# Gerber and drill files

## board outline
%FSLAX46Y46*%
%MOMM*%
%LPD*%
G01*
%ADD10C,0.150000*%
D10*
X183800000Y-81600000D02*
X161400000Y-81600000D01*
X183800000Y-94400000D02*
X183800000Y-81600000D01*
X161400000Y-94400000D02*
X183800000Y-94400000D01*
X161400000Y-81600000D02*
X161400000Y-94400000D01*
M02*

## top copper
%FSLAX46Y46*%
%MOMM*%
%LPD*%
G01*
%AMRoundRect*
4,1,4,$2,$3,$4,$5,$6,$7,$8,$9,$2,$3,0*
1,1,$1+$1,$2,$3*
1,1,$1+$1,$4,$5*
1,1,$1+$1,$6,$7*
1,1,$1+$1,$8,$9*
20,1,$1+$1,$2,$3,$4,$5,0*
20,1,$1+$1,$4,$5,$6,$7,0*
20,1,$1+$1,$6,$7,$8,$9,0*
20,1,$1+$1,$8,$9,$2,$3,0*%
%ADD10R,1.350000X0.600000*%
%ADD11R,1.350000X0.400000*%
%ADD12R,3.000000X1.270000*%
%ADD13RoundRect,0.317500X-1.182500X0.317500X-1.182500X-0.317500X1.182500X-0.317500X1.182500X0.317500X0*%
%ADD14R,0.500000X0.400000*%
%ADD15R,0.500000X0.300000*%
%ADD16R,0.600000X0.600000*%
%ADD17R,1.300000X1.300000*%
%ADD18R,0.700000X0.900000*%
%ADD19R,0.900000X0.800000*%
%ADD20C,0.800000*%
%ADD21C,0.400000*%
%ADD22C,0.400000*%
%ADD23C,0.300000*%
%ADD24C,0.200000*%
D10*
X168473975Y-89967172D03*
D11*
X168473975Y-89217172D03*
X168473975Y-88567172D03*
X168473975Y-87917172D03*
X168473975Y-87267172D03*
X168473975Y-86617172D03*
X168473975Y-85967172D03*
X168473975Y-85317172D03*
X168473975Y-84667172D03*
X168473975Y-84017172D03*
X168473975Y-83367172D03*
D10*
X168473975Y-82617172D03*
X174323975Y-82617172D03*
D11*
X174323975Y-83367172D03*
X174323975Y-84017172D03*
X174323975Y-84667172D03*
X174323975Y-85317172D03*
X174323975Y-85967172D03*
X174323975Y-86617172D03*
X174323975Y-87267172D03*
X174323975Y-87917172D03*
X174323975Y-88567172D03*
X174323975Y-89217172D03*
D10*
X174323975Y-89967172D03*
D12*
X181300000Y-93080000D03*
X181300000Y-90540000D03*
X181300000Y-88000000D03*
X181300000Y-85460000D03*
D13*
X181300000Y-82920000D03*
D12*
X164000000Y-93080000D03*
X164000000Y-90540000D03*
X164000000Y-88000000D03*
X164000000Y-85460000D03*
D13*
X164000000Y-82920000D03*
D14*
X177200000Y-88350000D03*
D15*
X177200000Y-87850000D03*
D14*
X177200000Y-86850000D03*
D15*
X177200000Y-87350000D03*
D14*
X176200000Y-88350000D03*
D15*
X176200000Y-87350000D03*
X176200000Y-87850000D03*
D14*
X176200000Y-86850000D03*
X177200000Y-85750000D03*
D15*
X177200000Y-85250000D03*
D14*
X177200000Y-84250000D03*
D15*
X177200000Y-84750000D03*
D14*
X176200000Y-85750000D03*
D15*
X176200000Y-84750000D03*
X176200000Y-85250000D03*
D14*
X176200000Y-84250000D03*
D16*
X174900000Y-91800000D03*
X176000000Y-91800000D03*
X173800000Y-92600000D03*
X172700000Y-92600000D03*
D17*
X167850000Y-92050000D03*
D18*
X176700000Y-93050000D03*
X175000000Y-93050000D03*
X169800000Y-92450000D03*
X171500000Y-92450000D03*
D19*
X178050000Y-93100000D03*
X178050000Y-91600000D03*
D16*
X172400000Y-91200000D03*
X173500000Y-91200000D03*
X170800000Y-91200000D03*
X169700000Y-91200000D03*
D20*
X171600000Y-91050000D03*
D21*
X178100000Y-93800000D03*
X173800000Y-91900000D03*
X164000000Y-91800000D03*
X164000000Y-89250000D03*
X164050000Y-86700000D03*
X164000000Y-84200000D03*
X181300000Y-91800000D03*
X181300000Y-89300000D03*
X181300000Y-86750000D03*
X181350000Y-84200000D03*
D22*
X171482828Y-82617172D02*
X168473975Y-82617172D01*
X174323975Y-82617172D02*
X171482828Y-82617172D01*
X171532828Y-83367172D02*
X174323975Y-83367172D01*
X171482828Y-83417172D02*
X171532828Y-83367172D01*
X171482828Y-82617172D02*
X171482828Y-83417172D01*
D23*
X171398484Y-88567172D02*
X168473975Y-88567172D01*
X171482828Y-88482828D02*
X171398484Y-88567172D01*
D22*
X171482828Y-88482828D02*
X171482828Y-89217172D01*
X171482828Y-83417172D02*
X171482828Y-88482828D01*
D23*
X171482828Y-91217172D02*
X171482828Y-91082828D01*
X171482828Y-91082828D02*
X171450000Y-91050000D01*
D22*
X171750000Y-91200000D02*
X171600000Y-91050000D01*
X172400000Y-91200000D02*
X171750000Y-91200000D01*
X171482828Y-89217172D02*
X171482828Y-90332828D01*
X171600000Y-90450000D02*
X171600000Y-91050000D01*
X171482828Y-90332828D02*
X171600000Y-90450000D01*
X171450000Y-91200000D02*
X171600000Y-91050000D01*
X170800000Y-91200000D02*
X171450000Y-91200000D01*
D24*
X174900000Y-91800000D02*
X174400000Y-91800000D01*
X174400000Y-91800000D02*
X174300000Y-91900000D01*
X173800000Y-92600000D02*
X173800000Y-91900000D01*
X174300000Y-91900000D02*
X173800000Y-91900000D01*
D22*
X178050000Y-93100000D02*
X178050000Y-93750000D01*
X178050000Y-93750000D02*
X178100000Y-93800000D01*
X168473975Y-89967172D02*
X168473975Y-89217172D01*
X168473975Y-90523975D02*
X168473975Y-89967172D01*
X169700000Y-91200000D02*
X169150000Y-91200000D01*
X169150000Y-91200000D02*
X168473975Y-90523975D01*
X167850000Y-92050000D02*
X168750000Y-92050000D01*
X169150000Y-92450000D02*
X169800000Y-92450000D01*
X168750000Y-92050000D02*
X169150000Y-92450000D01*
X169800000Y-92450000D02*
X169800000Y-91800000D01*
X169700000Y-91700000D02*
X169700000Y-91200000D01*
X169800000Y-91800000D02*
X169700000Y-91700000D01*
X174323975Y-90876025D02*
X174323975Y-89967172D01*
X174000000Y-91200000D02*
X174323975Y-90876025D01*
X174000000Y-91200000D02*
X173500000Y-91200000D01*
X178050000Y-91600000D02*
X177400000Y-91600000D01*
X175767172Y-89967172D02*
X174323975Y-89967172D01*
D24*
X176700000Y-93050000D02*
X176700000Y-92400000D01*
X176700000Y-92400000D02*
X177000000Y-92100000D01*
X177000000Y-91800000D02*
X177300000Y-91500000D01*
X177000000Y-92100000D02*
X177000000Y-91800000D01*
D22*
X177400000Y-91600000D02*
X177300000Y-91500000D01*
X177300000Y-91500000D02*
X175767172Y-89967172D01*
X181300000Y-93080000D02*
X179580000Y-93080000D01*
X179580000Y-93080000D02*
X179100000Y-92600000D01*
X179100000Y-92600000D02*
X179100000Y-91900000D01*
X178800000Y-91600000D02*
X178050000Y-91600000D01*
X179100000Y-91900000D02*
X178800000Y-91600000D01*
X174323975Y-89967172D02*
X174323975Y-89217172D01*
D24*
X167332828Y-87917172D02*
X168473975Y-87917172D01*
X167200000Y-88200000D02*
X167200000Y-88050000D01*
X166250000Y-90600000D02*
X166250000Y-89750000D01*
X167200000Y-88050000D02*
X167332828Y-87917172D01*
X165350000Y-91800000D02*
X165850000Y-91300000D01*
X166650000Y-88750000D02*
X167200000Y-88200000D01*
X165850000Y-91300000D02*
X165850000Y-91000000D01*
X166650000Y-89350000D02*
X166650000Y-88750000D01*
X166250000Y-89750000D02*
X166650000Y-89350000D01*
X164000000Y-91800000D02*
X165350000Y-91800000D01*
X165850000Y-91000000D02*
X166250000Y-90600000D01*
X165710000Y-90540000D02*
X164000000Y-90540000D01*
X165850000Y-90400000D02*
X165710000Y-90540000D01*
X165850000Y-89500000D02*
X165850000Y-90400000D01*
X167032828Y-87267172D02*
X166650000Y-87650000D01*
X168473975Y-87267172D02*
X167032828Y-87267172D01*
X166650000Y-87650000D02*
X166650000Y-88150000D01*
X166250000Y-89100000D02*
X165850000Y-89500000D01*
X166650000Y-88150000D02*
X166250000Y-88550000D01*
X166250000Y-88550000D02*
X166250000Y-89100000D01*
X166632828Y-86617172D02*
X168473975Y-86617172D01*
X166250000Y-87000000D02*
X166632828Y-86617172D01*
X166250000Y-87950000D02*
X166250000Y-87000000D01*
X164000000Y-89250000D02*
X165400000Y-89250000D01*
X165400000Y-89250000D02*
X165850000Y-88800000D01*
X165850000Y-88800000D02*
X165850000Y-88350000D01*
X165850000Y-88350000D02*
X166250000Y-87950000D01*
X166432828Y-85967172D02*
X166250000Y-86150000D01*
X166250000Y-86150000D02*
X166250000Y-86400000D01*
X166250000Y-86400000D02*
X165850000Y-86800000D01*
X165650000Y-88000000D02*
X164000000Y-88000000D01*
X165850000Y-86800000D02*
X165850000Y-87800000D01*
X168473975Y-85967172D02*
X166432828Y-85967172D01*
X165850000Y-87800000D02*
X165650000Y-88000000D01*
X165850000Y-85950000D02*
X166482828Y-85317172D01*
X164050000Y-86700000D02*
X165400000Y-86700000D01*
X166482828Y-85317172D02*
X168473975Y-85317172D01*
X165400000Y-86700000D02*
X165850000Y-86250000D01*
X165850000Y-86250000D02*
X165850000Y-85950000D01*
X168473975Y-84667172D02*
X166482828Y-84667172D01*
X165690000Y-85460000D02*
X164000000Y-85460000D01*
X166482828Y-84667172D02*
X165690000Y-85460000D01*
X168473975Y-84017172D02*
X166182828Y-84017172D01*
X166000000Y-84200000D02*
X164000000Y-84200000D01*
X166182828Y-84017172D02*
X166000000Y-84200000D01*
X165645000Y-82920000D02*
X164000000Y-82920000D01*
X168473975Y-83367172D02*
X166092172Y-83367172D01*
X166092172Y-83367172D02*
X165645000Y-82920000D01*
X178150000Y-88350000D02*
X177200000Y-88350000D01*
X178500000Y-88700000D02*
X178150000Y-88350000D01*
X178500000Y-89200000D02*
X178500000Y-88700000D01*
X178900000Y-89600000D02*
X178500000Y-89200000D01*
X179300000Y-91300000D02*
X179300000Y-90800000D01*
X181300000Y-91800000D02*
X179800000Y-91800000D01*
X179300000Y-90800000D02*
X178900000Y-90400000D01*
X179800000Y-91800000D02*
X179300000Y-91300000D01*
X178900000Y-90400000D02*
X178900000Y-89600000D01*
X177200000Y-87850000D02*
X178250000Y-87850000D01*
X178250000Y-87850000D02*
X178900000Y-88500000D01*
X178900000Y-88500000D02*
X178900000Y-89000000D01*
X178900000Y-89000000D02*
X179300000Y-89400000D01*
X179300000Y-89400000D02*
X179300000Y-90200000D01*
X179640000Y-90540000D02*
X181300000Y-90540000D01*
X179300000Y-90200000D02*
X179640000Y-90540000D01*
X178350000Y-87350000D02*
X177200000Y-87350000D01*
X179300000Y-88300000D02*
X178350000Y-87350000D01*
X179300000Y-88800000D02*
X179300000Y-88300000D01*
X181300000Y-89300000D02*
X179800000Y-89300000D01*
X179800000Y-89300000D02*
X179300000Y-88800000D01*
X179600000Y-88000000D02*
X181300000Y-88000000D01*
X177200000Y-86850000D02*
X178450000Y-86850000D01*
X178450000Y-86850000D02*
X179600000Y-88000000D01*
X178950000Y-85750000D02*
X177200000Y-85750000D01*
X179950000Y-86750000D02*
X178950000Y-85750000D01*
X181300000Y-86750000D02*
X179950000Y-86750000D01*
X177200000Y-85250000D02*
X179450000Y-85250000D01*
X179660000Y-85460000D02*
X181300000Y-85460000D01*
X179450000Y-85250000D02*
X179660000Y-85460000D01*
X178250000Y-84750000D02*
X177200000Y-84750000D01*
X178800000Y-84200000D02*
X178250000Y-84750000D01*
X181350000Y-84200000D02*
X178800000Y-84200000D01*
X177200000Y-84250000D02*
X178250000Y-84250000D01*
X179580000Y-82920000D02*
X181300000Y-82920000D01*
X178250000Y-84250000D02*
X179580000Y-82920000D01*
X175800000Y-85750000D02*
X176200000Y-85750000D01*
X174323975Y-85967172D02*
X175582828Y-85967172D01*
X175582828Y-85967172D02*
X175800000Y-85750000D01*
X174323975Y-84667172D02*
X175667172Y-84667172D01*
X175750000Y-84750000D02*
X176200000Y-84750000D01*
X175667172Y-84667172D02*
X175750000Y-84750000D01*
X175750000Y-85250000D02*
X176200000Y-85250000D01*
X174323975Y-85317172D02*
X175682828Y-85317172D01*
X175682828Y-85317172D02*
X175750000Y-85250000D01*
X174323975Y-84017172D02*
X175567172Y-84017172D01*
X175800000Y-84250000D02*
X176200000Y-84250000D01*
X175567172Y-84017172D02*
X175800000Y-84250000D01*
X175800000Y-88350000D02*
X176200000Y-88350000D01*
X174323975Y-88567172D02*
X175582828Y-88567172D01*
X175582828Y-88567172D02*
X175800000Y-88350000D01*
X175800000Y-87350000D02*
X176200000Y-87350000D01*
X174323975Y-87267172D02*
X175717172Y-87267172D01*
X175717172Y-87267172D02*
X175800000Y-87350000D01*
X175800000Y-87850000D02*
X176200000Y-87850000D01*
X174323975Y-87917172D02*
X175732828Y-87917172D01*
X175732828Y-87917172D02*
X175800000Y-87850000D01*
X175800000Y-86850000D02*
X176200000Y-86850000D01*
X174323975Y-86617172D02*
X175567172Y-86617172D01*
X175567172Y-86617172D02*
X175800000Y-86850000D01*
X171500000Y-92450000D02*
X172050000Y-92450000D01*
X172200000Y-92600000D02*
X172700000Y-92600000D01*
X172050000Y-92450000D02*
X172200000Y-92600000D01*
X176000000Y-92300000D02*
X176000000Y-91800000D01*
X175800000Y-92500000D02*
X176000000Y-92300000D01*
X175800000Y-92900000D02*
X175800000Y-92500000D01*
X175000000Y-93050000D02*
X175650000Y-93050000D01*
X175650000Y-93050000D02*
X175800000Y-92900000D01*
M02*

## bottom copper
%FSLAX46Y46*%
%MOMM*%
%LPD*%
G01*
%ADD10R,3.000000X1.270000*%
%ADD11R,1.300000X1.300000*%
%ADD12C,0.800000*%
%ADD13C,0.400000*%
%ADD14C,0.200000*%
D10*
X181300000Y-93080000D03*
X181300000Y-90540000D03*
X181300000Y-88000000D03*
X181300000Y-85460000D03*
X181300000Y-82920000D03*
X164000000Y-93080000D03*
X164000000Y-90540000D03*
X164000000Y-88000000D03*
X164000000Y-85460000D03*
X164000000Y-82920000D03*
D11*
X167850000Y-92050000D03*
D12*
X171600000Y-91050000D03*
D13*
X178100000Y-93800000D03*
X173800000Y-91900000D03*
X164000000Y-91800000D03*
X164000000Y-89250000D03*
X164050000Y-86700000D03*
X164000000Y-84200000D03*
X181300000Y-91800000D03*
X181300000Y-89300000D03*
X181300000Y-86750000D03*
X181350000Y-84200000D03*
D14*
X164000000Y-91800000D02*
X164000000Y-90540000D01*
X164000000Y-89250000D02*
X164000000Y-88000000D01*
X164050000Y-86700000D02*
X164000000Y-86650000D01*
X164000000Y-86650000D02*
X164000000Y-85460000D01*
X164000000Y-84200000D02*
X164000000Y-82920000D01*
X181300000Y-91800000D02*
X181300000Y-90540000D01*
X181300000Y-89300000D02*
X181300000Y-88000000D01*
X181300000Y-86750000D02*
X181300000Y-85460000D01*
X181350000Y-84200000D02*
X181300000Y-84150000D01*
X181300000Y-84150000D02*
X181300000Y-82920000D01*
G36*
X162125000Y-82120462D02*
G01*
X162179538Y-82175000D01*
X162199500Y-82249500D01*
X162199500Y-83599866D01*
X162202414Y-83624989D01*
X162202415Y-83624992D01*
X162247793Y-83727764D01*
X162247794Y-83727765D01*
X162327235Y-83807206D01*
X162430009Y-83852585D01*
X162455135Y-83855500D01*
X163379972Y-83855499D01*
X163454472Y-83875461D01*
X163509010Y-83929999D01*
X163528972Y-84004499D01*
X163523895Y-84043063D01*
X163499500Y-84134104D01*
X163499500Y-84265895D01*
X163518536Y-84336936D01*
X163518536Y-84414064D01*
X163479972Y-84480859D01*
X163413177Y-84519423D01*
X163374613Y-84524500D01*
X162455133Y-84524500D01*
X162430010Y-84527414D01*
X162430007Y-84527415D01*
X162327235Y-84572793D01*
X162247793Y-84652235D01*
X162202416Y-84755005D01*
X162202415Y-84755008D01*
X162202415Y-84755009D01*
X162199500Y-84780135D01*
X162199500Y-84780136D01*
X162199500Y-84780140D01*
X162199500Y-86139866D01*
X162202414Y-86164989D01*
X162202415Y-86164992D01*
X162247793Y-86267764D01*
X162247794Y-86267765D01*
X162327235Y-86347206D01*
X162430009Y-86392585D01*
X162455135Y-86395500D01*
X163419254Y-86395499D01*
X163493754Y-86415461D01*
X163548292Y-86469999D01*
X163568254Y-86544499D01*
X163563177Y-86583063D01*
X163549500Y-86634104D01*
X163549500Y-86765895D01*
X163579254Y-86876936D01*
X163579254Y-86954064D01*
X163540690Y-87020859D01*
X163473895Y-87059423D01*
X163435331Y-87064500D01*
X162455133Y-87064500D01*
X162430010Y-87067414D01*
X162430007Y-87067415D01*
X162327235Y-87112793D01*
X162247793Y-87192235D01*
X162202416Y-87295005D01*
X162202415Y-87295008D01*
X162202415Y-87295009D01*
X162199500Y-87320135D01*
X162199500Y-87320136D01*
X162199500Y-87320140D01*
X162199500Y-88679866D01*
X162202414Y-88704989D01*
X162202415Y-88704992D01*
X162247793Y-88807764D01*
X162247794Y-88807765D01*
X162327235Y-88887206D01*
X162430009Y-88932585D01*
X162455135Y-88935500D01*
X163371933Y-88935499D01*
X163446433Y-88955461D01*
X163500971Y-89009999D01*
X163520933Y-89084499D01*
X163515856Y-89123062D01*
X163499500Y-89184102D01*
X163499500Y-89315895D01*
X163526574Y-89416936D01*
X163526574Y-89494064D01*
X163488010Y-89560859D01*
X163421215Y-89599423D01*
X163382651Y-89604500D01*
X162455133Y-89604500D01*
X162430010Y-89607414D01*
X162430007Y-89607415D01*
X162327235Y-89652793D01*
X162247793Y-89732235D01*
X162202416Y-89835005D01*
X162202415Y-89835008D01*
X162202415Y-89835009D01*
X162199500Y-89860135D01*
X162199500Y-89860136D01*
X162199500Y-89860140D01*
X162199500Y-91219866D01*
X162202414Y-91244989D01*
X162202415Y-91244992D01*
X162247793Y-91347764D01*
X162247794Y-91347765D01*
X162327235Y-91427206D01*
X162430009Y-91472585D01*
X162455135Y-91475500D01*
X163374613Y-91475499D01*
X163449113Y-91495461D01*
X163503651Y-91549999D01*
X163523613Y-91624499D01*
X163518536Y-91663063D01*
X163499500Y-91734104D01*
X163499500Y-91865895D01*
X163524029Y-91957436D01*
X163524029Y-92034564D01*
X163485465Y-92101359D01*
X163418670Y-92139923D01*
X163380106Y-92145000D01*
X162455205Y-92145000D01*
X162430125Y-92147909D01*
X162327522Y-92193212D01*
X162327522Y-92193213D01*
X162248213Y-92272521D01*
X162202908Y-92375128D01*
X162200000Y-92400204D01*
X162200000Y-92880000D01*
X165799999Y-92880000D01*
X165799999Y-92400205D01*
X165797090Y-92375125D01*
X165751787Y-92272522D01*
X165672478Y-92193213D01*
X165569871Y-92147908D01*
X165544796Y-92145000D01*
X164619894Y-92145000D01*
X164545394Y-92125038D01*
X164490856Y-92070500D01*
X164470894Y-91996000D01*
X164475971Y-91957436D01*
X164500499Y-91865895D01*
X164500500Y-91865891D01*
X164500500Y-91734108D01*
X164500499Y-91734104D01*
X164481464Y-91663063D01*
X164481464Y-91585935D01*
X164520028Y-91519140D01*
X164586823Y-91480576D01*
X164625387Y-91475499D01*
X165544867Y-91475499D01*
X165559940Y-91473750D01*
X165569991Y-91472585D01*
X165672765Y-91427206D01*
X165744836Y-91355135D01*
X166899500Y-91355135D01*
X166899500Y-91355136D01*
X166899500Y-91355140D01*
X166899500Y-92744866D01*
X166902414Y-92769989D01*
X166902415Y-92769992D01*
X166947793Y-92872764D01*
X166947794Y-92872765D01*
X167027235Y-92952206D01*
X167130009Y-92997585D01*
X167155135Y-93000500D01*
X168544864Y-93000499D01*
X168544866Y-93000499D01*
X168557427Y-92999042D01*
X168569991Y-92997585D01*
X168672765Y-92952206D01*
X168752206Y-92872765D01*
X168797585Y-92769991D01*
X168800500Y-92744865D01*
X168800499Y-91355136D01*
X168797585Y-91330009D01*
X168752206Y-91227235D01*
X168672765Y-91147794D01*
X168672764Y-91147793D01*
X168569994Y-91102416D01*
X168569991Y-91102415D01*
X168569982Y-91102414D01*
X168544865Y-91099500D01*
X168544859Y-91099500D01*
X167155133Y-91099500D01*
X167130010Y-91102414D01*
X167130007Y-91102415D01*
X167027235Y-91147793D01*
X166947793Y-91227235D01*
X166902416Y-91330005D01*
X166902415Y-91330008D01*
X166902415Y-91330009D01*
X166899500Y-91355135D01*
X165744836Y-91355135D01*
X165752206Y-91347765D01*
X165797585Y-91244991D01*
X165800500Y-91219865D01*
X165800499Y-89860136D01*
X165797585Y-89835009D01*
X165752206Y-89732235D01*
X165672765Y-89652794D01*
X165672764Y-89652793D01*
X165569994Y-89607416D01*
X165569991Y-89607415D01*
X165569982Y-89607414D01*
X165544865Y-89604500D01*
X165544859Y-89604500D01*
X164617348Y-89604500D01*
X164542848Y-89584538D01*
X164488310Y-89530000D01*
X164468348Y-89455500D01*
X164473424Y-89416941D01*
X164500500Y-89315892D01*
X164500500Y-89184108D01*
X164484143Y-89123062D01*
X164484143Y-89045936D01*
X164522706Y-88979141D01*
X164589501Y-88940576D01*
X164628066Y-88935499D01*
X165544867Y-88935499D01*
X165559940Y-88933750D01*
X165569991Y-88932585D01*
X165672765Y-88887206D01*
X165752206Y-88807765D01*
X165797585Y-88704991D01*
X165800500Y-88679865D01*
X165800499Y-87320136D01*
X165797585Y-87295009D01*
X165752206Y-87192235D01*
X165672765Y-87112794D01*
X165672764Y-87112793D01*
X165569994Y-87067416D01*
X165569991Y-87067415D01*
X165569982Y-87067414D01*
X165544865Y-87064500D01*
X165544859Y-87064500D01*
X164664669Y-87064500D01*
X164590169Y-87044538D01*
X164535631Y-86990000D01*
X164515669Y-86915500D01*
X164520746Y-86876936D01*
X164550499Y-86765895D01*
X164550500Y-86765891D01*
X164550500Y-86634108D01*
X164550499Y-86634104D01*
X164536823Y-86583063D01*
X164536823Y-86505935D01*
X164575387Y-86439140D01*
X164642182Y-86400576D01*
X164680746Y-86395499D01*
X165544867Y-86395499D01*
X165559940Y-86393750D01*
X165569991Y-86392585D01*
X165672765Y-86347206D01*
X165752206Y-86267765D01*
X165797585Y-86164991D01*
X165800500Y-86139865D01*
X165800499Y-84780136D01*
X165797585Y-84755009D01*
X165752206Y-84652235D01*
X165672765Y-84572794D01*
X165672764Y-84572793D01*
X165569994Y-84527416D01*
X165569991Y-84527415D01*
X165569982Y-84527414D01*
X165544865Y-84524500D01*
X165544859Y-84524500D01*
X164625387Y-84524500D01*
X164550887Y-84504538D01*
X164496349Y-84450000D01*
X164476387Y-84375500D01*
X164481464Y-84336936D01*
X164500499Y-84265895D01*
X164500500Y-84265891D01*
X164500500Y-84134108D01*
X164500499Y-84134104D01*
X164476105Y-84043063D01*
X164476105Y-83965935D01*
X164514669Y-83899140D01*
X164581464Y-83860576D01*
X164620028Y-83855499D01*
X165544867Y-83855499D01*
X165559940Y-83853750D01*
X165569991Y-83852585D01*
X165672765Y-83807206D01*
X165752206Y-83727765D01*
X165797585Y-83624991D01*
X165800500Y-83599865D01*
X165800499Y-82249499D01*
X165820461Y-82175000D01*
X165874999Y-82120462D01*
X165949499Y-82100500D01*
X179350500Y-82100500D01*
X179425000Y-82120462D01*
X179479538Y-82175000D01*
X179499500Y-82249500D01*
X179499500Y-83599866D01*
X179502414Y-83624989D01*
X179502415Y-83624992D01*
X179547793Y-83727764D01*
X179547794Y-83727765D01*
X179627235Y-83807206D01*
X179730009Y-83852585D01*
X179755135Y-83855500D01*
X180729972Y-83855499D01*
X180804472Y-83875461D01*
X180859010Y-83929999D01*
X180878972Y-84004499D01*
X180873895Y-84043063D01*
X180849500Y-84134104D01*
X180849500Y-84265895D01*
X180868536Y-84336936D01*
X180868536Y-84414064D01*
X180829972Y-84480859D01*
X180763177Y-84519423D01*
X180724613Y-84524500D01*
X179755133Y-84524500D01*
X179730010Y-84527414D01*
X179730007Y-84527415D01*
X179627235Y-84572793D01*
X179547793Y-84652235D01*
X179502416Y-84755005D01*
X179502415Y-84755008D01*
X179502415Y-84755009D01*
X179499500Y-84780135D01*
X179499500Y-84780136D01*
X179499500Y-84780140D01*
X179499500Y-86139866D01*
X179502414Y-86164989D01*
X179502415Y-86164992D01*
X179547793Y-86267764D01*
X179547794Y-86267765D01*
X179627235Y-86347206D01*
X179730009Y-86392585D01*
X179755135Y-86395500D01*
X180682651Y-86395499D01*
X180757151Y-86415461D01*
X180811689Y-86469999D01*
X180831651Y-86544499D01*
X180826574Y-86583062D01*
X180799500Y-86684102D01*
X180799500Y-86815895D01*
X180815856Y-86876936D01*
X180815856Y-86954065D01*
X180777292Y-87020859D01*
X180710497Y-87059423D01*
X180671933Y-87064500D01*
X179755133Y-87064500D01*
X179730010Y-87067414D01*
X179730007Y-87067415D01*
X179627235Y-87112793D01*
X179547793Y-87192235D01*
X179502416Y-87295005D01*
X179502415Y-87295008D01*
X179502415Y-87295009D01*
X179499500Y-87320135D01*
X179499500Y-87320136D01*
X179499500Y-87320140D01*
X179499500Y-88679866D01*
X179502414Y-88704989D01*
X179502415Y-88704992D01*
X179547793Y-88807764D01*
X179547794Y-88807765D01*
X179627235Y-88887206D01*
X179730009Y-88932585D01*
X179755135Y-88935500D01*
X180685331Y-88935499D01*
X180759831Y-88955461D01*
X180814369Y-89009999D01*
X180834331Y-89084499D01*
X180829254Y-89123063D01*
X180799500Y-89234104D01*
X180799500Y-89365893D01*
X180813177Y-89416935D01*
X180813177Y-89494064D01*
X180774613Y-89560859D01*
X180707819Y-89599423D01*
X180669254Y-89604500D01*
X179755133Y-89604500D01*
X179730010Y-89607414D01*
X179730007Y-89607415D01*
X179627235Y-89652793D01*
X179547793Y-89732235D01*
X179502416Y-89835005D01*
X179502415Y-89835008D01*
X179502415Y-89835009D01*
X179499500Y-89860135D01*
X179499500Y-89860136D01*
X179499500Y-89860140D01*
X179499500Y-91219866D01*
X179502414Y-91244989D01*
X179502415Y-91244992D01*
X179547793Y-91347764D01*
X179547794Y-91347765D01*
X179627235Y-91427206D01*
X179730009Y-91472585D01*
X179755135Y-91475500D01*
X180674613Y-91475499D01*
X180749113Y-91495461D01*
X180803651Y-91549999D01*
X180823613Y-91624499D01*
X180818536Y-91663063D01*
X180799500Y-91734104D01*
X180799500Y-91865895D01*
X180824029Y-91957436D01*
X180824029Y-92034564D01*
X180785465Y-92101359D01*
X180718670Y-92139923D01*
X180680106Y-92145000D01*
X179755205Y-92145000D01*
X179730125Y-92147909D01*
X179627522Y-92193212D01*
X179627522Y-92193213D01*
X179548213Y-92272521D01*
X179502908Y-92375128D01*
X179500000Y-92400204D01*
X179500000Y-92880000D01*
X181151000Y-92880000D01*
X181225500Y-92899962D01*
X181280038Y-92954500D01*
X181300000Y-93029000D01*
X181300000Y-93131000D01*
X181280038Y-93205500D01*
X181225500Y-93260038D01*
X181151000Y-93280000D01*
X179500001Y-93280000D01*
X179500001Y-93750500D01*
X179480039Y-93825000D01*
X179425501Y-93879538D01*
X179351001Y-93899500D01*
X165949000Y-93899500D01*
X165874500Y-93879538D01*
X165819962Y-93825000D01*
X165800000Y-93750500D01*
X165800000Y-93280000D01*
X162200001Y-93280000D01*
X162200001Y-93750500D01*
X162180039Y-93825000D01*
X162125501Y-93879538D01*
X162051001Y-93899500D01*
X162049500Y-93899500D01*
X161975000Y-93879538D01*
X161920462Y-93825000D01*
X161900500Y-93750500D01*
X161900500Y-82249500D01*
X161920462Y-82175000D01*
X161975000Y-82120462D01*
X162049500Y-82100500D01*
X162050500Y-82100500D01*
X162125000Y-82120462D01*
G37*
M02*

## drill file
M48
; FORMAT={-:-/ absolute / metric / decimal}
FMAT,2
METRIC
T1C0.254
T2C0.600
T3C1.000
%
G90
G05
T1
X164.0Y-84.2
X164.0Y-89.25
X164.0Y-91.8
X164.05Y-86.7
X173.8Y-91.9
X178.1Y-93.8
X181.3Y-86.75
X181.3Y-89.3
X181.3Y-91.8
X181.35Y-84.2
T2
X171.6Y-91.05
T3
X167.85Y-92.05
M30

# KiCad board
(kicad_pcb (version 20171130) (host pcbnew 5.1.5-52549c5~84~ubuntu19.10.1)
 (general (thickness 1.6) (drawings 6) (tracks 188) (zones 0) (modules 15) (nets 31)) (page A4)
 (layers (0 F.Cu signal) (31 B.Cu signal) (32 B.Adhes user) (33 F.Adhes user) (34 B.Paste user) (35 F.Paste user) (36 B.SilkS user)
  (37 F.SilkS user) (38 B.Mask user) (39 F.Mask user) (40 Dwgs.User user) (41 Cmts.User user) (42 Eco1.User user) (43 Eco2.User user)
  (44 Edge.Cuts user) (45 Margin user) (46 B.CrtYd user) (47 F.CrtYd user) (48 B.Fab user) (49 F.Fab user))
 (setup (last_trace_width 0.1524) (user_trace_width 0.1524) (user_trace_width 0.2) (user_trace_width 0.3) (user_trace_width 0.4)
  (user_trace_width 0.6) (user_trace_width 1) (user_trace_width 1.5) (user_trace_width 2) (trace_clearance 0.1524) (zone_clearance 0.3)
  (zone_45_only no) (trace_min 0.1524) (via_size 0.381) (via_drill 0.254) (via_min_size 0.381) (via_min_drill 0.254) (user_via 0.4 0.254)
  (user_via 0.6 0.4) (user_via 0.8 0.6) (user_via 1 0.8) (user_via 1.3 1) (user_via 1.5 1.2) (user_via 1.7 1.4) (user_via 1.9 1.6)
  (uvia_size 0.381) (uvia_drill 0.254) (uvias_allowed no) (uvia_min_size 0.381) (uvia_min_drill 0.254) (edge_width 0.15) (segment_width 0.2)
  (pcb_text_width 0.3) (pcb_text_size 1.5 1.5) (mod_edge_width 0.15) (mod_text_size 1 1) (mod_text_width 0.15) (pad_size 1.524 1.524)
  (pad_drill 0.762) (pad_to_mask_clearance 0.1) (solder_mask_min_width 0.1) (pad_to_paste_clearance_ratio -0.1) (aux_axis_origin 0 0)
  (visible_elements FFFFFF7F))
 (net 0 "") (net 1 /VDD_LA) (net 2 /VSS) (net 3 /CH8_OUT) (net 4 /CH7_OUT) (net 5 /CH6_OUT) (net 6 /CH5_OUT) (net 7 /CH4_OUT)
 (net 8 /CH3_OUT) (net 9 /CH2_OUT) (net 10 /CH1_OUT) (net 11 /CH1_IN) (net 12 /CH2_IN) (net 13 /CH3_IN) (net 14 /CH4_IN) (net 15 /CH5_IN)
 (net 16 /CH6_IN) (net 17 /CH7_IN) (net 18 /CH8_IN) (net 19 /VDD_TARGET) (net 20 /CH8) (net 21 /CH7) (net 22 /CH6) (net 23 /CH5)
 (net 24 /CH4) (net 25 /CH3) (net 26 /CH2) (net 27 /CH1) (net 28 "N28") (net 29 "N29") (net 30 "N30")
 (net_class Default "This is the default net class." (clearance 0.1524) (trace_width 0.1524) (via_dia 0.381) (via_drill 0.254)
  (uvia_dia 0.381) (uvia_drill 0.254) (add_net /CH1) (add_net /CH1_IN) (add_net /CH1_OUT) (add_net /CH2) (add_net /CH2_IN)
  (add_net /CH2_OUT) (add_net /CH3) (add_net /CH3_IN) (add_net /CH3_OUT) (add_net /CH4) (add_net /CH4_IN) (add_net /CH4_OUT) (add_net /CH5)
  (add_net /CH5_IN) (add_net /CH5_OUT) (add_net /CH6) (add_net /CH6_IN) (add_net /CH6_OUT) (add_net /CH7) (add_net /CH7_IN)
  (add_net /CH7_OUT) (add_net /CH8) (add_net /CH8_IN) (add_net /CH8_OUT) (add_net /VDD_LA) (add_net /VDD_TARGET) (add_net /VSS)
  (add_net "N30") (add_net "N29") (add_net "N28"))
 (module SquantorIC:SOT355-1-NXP (layer F.Cu) (at 171.35 86.25 180)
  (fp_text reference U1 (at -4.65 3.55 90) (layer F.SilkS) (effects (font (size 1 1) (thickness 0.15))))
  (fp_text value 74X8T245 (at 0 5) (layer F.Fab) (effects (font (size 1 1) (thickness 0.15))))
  (pad 24 smd rect (at 2.876025 -3.717172 90) (size 0.6 1.35) (layers F.Cu F.Paste F.Mask) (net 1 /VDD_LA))
  (pad 23 smd rect (at 2.876025 -2.967172 90) (size 0.4 1.35) (layers F.Cu F.Paste F.Mask) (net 1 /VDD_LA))
  (pad 22 smd rect (at 2.876025 -2.317172 90) (size 0.4 1.35) (layers F.Cu F.Paste F.Mask) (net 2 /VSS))
  (pad 21 smd rect (at 2.876025 -1.667172 90) (size 0.4 1.35) (layers F.Cu F.Paste F.Mask) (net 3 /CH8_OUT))
  (pad 20 smd rect (at 2.876025 -1.017172 90) (size 0.4 1.35) (layers F.Cu F.Paste F.Mask) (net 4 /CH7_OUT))
  (pad 19 smd rect (at 2.876025 -0.367172 90) (size 0.4 1.35) (layers F.Cu F.Paste F.Mask) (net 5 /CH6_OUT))
  (pad 18 smd rect (at 2.876025 0.282828 90) (size 0.4 1.35) (layers F.Cu F.Paste F.Mask) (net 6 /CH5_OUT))
  (pad 17 smd rect (at 2.876025 0.932828 90) (size 0.4 1.35) (layers F.Cu F.Paste F.Mask) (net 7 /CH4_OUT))
  (pad 16 smd rect (at 2.876025 1.582828 90) (size 0.4 1.35) (layers F.Cu F.Paste F.Mask) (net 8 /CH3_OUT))
  (pad 15 smd rect (at 2.876025 2.232828 90) (size 0.4 1.35) (layers F.Cu F.Paste F.Mask) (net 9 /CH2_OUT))
  (pad 14 smd rect (at 2.876025 2.882828 90) (size 0.4 1.35) (layers F.Cu F.Paste F.Mask) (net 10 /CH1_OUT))
  (pad 13 smd rect (at 2.876025 3.632828 90) (size 0.6 1.35) (layers F.Cu F.Paste F.Mask) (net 2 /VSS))
  (pad 12 smd rect (at -2.973975 3.632828 90) (size 0.6 1.35) (layers F.Cu F.Paste F.Mask) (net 2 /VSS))
  (pad 11 smd rect (at -2.973975 2.882828 90) (size 0.4 1.35) (layers F.Cu F.Paste F.Mask) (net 2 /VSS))
  (pad 10 smd rect (at -2.973975 2.232828 90) (size 0.4 1.35) (layers F.Cu F.Paste F.Mask) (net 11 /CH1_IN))
  (pad 9 smd rect (at -2.973975 1.582828 90) (size 0.4 1.35) (layers F.Cu F.Paste F.Mask) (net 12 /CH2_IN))
  (pad 8 smd rect (at -2.973975 0.932828 90) (size 0.4 1.35) (layers F.Cu F.Paste F.Mask) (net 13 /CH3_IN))
  (pad 7 smd rect (at -2.973975 0.282828 90) (size 0.4 1.35) (layers F.Cu F.Paste F.Mask) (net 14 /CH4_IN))
  (pad 6 smd rect (at -2.973975 -0.367172 90) (size 0.4 1.35) (layers F.Cu F.Paste F.Mask) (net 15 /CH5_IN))
  (pad 5 smd rect (at -2.973975 -1.017172 90) (size 0.4 1.35) (layers F.Cu F.Paste F.Mask) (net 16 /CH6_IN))
  (pad 4 smd rect (at -2.973975 -1.667172 90) (size 0.4 1.35) (layers F.Cu F.Paste F.Mask) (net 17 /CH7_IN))
  (pad 3 smd rect (at -2.973975 -2.317172 90) (size 0.4 1.35) (layers F.Cu F.Paste F.Mask) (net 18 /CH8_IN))
  (pad 2 smd rect (at -2.973975 -2.967172 90) (size 0.4 1.35) (layers F.Cu F.Paste F.Mask) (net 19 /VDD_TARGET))
  (pad 1 smd rect (at -2.973975 -3.717172 90) (size 0.6 1.35) (layers F.Cu F.Paste F.Mask) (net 19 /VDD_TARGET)))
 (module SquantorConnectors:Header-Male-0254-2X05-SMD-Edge (layer B.Cu) (at 183.84 88 270)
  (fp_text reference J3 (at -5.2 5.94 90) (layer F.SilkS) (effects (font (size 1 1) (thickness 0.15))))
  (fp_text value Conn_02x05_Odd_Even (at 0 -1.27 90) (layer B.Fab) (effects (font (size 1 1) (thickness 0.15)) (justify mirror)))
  (pad 10 smd rect (at 5.08 2.54 270) (size 1.27 3) (layers B.Cu B.Paste B.Mask) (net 2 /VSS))
  (pad 9 smd rect (at 5.08 2.54 270) (size 1.27 3) (layers F.Cu F.Paste F.Mask) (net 19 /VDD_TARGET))
  (pad 8 smd rect (at 2.54 2.54 270) (size 1.27 3) (layers B.Cu B.Paste B.Mask) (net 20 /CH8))
  (pad 7 smd rect (at 2.54 2.54 270) (size 1.27 3) (layers F.Cu F.Paste F.Mask) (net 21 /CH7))
  (pad 6 smd rect (at 0 2.54 270) (size 1.27 3) (layers B.Cu B.Paste B.Mask) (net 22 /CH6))
  (pad 5 smd rect (at 0 2.54 270) (size 1.27 3) (layers F.Cu F.Paste F.Mask) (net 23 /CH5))
  (pad 4 smd rect (at -2.54 2.54 270) (size 1.27 3) (layers B.Cu B.Paste B.Mask) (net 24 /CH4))
  (pad 3 smd rect (at -2.54 2.54 270) (size 1.27 3) (layers F.Cu F.Paste F.Mask) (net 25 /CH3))
  (pad 2 smd rect (at -5.08 2.54 270) (size 1.27 3) (layers B.Cu B.Paste B.Mask) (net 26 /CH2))
  (pad 1 smd roundrect (at -5.08 2.54 270) (size 1.27 3) (layers F.Cu F.Paste F.Mask) (roundrect_rratio 0.25) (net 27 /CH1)))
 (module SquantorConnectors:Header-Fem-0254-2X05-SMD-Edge (layer F.Cu) (at 161.46 88 270)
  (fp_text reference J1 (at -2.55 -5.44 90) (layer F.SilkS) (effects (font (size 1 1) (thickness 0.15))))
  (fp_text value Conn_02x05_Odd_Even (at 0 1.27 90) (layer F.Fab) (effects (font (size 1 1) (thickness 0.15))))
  (pad 10 smd rect (at 5.08 -2.54 270) (size 1.27 3) (layers B.Cu B.Paste B.Mask) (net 2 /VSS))
  (pad 9 smd rect (at 5.08 -2.54 270) (size 1.27 3) (layers F.Cu F.Paste F.Mask) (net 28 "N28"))
  (pad 8 smd rect (at 2.54 -2.54 270) (size 1.27 3) (layers B.Cu B.Paste B.Mask) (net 3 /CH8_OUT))
  (pad 7 smd rect (at 2.54 -2.54 270) (size 1.27 3) (layers F.Cu F.Paste F.Mask) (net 4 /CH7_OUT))
  (pad 6 smd rect (at 0 -2.54 270) (size 1.27 3) (layers B.Cu B.Paste B.Mask) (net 5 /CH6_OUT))
  (pad 5 smd rect (at 0 -2.54 270) (size 1.27 3) (layers F.Cu F.Paste F.Mask) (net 6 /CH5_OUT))
  (pad 4 smd rect (at -2.54 -2.54 270) (size 1.27 3) (layers B.Cu B.Paste B.Mask) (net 7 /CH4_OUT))
  (pad 3 smd rect (at -2.54 -2.54 270) (size 1.27 3) (layers F.Cu F.Paste F.Mask) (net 8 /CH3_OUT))
  (pad 2 smd rect (at -5.08 -2.54 270) (size 1.27 3) (layers B.Cu B.Paste B.Mask) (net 9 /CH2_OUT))
  (pad 1 smd roundrect (at -5.08 -2.54 270) (size 1.27 3) (layers F.Cu F.Paste F.Mask) (roundrect_rratio 0.25) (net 10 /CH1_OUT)))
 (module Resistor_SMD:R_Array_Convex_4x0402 (layer F.Cu) (at 176.7 87.6)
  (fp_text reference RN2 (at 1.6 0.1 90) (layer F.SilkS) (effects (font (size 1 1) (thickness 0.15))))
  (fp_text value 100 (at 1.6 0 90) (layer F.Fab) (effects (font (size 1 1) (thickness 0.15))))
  (pad 5 smd rect (at 0.5 0.75) (size 0.5 0.4) (layers F.Cu F.Paste F.Mask) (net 20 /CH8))
  (pad 6 smd rect (at 0.5 0.25) (size 0.5 0.3) (layers F.Cu F.Paste F.Mask) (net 21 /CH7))
  (pad 8 smd rect (at 0.5 -0.75) (size 0.5 0.4) (layers F.Cu F.Paste F.Mask) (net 23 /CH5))
  (pad 7 smd rect (at 0.5 -0.25) (size 0.5 0.3) (layers F.Cu F.Paste F.Mask) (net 22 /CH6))
  (pad 4 smd rect (at -0.5 0.75) (size 0.5 0.4) (layers F.Cu F.Paste F.Mask) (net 18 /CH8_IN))
  (pad 2 smd rect (at -0.5 -0.25) (size 0.5 0.3) (layers F.Cu F.Paste F.Mask) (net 16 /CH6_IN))
  (pad 3 smd rect (at -0.5 0.25) (size 0.5 0.3) (layers F.Cu F.Paste F.Mask) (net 17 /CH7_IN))
  (pad 1 smd rect (at -0.5 -0.75) (size 0.5 0.4) (layers F.Cu F.Paste F.Mask) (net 15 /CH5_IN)))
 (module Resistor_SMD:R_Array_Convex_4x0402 (layer F.Cu) (at 176.7 85)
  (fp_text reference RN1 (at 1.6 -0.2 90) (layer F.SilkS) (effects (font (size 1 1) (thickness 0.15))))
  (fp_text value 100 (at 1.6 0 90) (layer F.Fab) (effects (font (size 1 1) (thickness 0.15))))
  (pad 5 smd rect (at 0.5 0.75) (size 0.5 0.4) (layers F.Cu F.Paste F.Mask) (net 24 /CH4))
  (pad 6 smd rect (at 0.5 0.25) (size 0.5 0.3) (layers F.Cu F.Paste F.Mask) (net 25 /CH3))
  (pad 8 smd rect (at 0.5 -0.75) (size 0.5 0.4) (layers F.Cu F.Paste F.Mask) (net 27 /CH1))
  (pad 7 smd rect (at 0.5 -0.25) (size 0.5 0.3) (layers F.Cu F.Paste F.Mask) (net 26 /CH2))
  (pad 4 smd rect (at -0.5 0.75) (size 0.5 0.4) (layers F.Cu F.Paste F.Mask) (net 14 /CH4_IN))
  (pad 2 smd rect (at -0.5 -0.25) (size 0.5 0.3) (layers F.Cu F.Paste F.Mask) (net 12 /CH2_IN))
  (pad 3 smd rect (at -0.5 0.25) (size 0.5 0.3) (layers F.Cu F.Paste F.Mask) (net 13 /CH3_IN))
  (pad 1 smd rect (at -0.5 -0.75) (size 0.5 0.4) (layers F.Cu F.Paste F.Mask) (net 11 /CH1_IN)))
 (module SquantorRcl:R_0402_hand (layer F.Cu) (at 175.45 91.8 180)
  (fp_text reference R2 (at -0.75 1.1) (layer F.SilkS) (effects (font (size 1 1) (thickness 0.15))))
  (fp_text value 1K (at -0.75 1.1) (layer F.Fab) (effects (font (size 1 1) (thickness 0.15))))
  (pad 2 smd rect (at 0.55 0 180) (size 0.6 0.6) (layers F.Cu F.Paste F.Mask) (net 2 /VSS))
  (pad 1 smd rect (at -0.55 0 180) (size 0.6 0.6) (layers F.Cu F.Paste F.Mask) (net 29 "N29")))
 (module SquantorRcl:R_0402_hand (layer F.Cu) (at 173.25 92.6)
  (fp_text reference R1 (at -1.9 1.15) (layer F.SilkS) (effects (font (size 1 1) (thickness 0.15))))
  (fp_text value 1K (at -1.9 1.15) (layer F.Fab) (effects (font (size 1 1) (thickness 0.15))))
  (pad 2 smd rect (at 0.55 0) (size 0.6 0.6) (layers F.Cu F.Paste F.Mask) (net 2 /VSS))
  (pad 1 smd rect (at -0.55 0) (size 0.6 0.6) (layers F.Cu F.Paste F.Mask) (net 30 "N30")))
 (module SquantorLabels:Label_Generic (layer B.Cu) (at 173 90 180)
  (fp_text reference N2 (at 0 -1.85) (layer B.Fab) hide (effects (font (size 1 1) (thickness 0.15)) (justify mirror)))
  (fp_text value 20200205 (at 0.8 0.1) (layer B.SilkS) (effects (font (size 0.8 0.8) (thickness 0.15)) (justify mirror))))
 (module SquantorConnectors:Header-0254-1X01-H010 (layer F.Cu) (at 167.85 92.05)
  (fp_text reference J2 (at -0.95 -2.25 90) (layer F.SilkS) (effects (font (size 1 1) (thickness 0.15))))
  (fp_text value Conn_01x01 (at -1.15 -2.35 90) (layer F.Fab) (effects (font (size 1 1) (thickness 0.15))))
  (pad 1 thru_hole rect (at 0 0 180) (size 1.3 1.3) (drill 1) (layers *.Cu *.Mask) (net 1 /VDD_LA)))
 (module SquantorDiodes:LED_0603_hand (layer F.Cu) (at 175.85 93.05)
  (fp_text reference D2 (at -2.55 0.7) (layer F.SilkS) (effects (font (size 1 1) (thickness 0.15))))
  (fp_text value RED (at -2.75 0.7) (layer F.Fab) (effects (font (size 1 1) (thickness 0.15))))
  (pad 2 smd rect (at 0.85 0) (size 0.7 0.9) (layers F.Cu F.Paste F.Mask) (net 19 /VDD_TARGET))
  (pad 1 smd rect (at -0.85 0) (size 0.7 0.9) (layers F.Cu F.Paste F.Mask) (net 29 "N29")))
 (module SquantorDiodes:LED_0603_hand (layer F.Cu) (at 170.65 92.45 180)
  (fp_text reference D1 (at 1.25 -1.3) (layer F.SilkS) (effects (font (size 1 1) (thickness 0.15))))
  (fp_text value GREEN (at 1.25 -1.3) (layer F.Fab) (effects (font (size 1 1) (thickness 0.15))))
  (pad 2 smd rect (at 0.85 0 180) (size 0.7 0.9) (layers F.Cu F.Paste F.Mask) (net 1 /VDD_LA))
  (pad 1 smd rect (at -0.85 0 180) (size 0.7 0.9) (layers F.Cu F.Paste F.Mask) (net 30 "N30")))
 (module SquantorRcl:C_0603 (layer F.Cu) (at 178.05 92.35 270)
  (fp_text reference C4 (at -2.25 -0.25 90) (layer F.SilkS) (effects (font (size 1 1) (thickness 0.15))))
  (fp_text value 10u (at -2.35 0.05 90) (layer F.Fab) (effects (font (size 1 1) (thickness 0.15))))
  (pad 2 smd rect (at 0.75 0 270) (size 0.8 0.9) (layers F.Cu F.Paste F.Mask) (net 2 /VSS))
  (pad 1 smd rect (at -0.75 0 270) (size 0.8 0.9) (layers F.Cu F.Paste F.Mask) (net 19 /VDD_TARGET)))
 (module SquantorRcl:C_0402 (layer F.Cu) (at 172.95 91.2 180)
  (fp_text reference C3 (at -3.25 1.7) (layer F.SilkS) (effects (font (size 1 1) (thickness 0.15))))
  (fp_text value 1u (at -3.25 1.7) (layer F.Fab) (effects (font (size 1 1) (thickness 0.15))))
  (pad 2 smd rect (at 0.55 0 180) (size 0.6 0.6) (layers F.Cu F.Paste F.Mask) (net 2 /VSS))
  (pad 1 smd rect (at -0.55 0 180) (size 0.6 0.6) (layers F.Cu F.Paste F.Mask) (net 19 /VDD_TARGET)))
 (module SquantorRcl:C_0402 (layer F.Cu) (at 170.25 91.2)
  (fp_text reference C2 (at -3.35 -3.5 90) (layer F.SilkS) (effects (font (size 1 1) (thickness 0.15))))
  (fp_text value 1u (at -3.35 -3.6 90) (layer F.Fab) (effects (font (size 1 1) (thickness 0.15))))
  (pad 2 smd rect (at 0.55 0) (size 0.6 0.6) (layers F.Cu F.Paste F.Mask) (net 2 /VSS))
  (pad 1 smd rect (at -0.55 0) (size 0.6 0.6) (layers F.Cu F.Paste F.Mask) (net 1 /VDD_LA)))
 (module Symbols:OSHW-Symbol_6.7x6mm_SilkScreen (layer B.Cu) (at 172.5 86 180)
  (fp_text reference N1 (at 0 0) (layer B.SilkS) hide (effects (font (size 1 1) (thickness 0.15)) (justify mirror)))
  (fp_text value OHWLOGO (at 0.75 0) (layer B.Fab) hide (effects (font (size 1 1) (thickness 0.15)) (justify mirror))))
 (gr_line (start 183.8 81.6) (end 161.4 81.6) (layer Edge.Cuts) (width 0.15))
 (gr_line (start 183.8 94.4) (end 183.8 81.6) (layer Edge.Cuts) (width 0.15))
 (gr_line (start 161.4 94.4) (end 183.8 94.4) (layer Edge.Cuts) (width 0.15))
 (gr_line (start 161.4 81.6) (end 161.4 94.4) (layer Edge.Cuts) (width 0.15))
 (segment (start 171.482828 82.617172) (end 168.473975 82.617172) (width 0.4) (layer F.Cu) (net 2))
 (segment (start 174.323975 82.617172) (end 171.482828 82.617172) (width 0.4) (layer F.Cu) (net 2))
 (segment (start 171.532828 83.367172) (end 174.323975 83.367172) (width 0.4) (layer F.Cu) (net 2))
 (segment (start 171.482828 83.417172) (end 171.532828 83.367172) (width 0.4) (layer F.Cu) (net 2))
 (segment (start 171.482828 82.617172) (end 171.482828 83.417172) (width 0.4) (layer F.Cu) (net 2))
 (segment (start 171.398484 88.567172) (end 168.473975 88.567172) (width 0.3) (layer F.Cu) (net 2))
 (segment (start 171.482828 88.482828) (end 171.398484 88.567172) (width 0.3) (layer F.Cu) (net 2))
 (segment (start 171.482828 88.482828) (end 171.482828 89.217172) (width 0.4) (layer F.Cu) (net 2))
 (segment (start 171.482828 83.417172) (end 171.482828 88.482828) (width 0.4) (layer F.Cu) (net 2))
 (via (at 171.6 91.05) (size 0.8) (drill 0.6) (layers F.Cu B.Cu) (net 2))
 (segment (start 171.482828 91.217172) (end 171.482828 91.082828) (width 0.3) (layer F.Cu) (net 2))
 (segment (start 171.482828 91.082828) (end 171.45 91.05) (width 0.3) (layer F.Cu) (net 2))
 (segment (start 171.75 91.2) (end 171.6 91.05) (width 0.4) (layer F.Cu) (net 2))
 (segment (start 172.4 91.2) (end 171.75 91.2) (width 0.4) (layer F.Cu) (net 2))
 (segment (start 171.482828 89.217172) (end 171.482828 90.332828) (width 0.4) (layer F.Cu) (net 2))
 (segment (start 171.6 90.45) (end 171.6 91.05) (width 0.4) (layer F.Cu) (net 2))
 (segment (start 171.482828 90.332828) (end 171.6 90.45) (width 0.4) (layer F.Cu) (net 2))
 (segment (start 171.45 91.2) (end 171.6 91.05) (width 0.4) (layer F.Cu) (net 2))
 (segment (start 170.8 91.2) (end 171.45 91.2) (width 0.4) (layer F.Cu) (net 2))
 (segment (start 174.9 91.8) (end 174.4 91.8) (width 0.2) (layer F.Cu) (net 2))
 (segment (start 174.4 91.8) (end 174.3 91.9) (width 0.2) (layer F.Cu) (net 2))
 (segment (start 173.8 92.6) (end 173.8 91.9) (width 0.2) (layer F.Cu) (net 2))
 (segment (start 174.3 91.9) (end 173.8 91.9) (width 0.2) (layer F.Cu) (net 2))
 (via (at 178.1 93.8) (size 0.4) (drill 0.254) (layers F.Cu B.Cu) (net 2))
 (segment (start 178.05 93.1) (end 178.05 93.75) (width 0.4) (layer F.Cu) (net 2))
 (segment (start 178.05 93.75) (end 178.1 93.8) (width 0.4) (layer F.Cu) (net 2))
 (via (at 173.8 91.9) (size 0.4) (drill 0.254) (layers F.Cu B.Cu) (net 2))
 (segment (start 168.473975 89.967172) (end 168.473975 89.217172) (width 0.4) (layer F.Cu) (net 1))
 (segment (start 168.473975 90.523975) (end 168.473975 89.967172) (width 0.4) (layer F.Cu) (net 1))
 (segment (start 169.7 91.2) (end 169.15 91.2) (width 0.4) (layer F.Cu) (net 1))
 (segment (start 169.15 91.2) (end 168.473975 90.523975) (width 0.4) (layer F.Cu) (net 1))
 (segment (start 167.85 92.05) (end 168.75 92.05) (width 0.4) (layer F.Cu) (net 1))
 (segment (start 169.15 92.45) (end 169.8 92.45) (width 0.4) (layer F.Cu) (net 1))
 (segment (start 168.75 92.05) (end 169.15 92.45) (width 0.4) (layer F.Cu) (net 1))
 (segment (start 169.8 92.45) (end 169.8 91.8) (width 0.4) (layer F.Cu) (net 1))
 (segment (start 169.7 91.7) (end 169.7 91.2) (width 0.4) (layer F.Cu) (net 1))
 (segment (start 169.8 91.8) (end 169.7 91.7) (width 0.4) (layer F.Cu) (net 1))
 (segment (start 174.323975 90.876025) (end 174.323975 89.967172) (width 0.4) (layer F.Cu) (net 19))
 (segment (start 174 91.2) (end 174.323975 90.876025) (width 0.4) (layer F.Cu) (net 19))
 (segment (start 174 91.2) (end 173.5 91.2) (width 0.4) (layer F.Cu) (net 19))
 (segment (start 178.05 91.6) (end 177.4 91.6) (width 0.4) (layer F.Cu) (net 19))
 (segment (start 175.767172 89.967172) (end 174.323975 89.967172) (width 0.4) (layer F.Cu) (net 19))
 (segment (start 176.7 93.05) (end 176.7 92.4) (width 0.2) (layer F.Cu) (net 19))
 (segment (start 176.7 92.4) (end 177 92.1) (width 0.2) (layer F.Cu) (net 19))
 (segment (start 177 91.8) (end 177.3 91.5) (width 0.2) (layer F.Cu) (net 19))
 (segment (start 177 92.1) (end 177 91.8) (width 0.2) (layer F.Cu) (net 19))
 (segment (start 177.4 91.6) (end 177.3 91.5) (width 0.4) (layer F.Cu) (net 19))
 (segment (start 177.3 91.5) (end 175.767172 89.967172) (width 0.4) (layer F.Cu) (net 19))
 (segment (start 181.3 93.08) (end 179.58 93.08) (width 0.4) (layer F.Cu) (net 19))
 (segment (start 179.58 93.08) (end 179.1 92.6) (width 0.4) (layer F.Cu) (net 19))
 (segment (start 179.1 92.6) (end 179.1 91.9) (width 0.4) (layer F.Cu) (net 19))
 (segment (start 178.8 91.6) (end 178.05 91.6) (width 0.4) (layer F.Cu) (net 19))
 (segment (start 179.1 91.9) (end 178.8 91.6) (width 0.4) (layer F.Cu) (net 19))
 (segment (start 174.323975 89.967172) (end 174.323975 89.217172) (width 0.4) (layer F.Cu) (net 19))
 (segment (start 167.332828 87.917172) (end 168.473975 87.917172) (width 0.2) (layer F.Cu) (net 3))
 (segment (start 167.2 88.2) (end 167.2 88.05) (width 0.2) (layer F.Cu) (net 3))
 (segment (start 166.25 90.6) (end 166.25 89.75) (width 0.2) (layer F.Cu) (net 3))
 (segment (start 164 91.8) (end 164 90.54) (width 0.2) (layer B.Cu) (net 3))
 (segment (start 167.2 88.05) (end 167.332828 87.917172) (width 0.2) (layer F.Cu) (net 3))
 (via (at 164 91.8) (size 0.4) (drill 0.254) (layers F.Cu B.Cu) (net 3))
 (segment (start 165.35 91.8) (end 165.85 91.3) (width 0.2) (layer F.Cu) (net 3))
 (segment (start 166.65 88.75) (end 167.2 88.2) (width 0.2) (layer F.Cu) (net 3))
 (segment (start 165.85 91.3) (end 165.85 91) (width 0.2) (layer F.Cu) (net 3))
 (segment (start 166.65 89.35) (end 166.65 88.75) (width 0.2) (layer F.Cu) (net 3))
 (segment (start 166.25 89.75) (end 166.65 89.35) (width 0.2) (layer F.Cu) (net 3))
 (segment (start 164 91.8) (end 165.35 91.8) (width 0.2) (layer F.Cu) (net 3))
 (segment (start 165.85 91) (end 166.25 90.6) (width 0.2) (layer F.Cu) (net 3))
 (segment (start 165.71 90.54) (end 164 90.54) (width 0.2) (layer F.Cu) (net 4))
 (segment (start 165.85 90.4) (end 165.71 90.54) (width 0.2) (layer F.Cu) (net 4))
 (segment (start 165.85 89.5) (end 165.85 90.4) (width 0.2) (layer F.Cu) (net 4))
 (segment (start 167.032828 87.267172) (end 166.65 87.65) (width 0.2) (layer F.Cu) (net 4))
 (segment (start 168.473975 87.267172) (end 167.032828 87.267172) (width 0.2) (layer F.Cu) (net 4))
 (segment (start 166.65 87.65) (end 166.65 88.15) (width 0.2) (layer F.Cu) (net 4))
 (segment (start 166.25 89.1) (end 165.85 89.5) (width 0.2) (layer F.Cu) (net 4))
 (segment (start 166.65 88.15) (end 166.25 88.55) (width 0.2) (layer F.Cu) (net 4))
 (segment (start 166.25 88.55) (end 166.25 89.1) (width 0.2) (layer F.Cu) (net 4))
 (segment (start 166.632828 86.617172) (end 168.473975 86.617172) (width 0.2) (layer F.Cu) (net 5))
 (segment (start 166.25 87) (end 166.632828 86.617172) (width 0.2) (layer F.Cu) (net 5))
 (segment (start 166.25 87.95) (end 166.25 87) (width 0.2) (layer F.Cu) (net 5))
 (segment (start 164 89.25) (end 164 88) (width 0.2) (layer B.Cu) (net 5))
 (via (at 164 89.25) (size 0.4) (drill 0.254) (layers F.Cu B.Cu) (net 5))
 (segment (start 164 89.25) (end 165.4 89.25) (width 0.2) (layer F.Cu) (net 5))
 (segment (start 165.4 89.25) (end 165.85 88.8) (width 0.2) (layer F.Cu) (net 5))
 (segment (start 165.85 88.8) (end 165.85 88.35) (width 0.2) (layer F.Cu) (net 5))
 (segment (start 165.85 88.35) (end 166.25 87.95) (width 0.2) (layer F.Cu) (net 5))
 (segment (start 166.432828 85.967172) (end 166.25 86.15) (width 0.2) (layer F.Cu) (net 6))
 (segment (start 166.25 86.15) (end 166.25 86.4) (width 0.2) (layer F.Cu) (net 6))
 (segment (start 166.25 86.4) (end 165.85 86.8) (width 0.2) (layer F.Cu) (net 6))
 (segment (start 165.65 88) (end 164 88) (width 0.2) (layer F.Cu) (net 6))
 (segment (start 165.85 86.8) (end 165.85 87.8) (width 0.2) (layer F.Cu) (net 6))
 (segment (start 168.473975 85.967172) (end 166.432828 85.967172) (width 0.2) (layer F.Cu) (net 6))
 (segment (start 165.85 87.8) (end 165.65 88) (width 0.2) (layer F.Cu) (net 6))
 (segment (start 165.85 85.95) (end 166.482828 85.317172) (width 0.2) (layer F.Cu) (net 7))
 (segment (start 164.05 86.7) (end 164 86.65) (width 0.2) (layer B.Cu) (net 7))
 (via (at 164.05 86.7) (size 0.4) (drill 0.254) (layers F.Cu B.Cu) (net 7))
 (segment (start 164.05 86.7) (end 165.4 86.7) (width 0.2) (layer F.Cu) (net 7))
 (segment (start 166.482828 85.317172) (end 168.473975 85.317172) (width 0.2) (layer F.Cu) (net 7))
 (segment (start 164 86.65) (end 164 85.46) (width 0.2) (layer B.Cu) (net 7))
 (segment (start 165.4 86.7) (end 165.85 86.25) (width 0.2) (layer F.Cu) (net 7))
 (segment (start 165.85 86.25) (end 165.85 85.95) (width 0.2) (layer F.Cu) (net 7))
 (segment (start 168.473975 84.667172) (end 166.482828 84.667172) (width 0.2) (layer F.Cu) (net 8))
 (segment (start 165.69 85.46) (end 164 85.46) (width 0.2) (layer F.Cu) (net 8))
 (segment (start 166.482828 84.667172) (end 165.69 85.46) (width 0.2) (layer F.Cu) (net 8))
 (via (at 164 84.2) (size 0.4) (drill 0.254) (layers F.Cu B.Cu) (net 9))
 (segment (start 164 84.2) (end 164 82.92) (width 0.2) (layer B.Cu) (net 9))
 (segment (start 168.473975 84.017172) (end 166.182828 84.017172) (width 0.2) (layer F.Cu) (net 9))
 (segment (start 166 84.2) (end 164 84.2) (width 0.2) (layer F.Cu) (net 9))
 (segment (start 166.182828 84.017172) (end 166 84.2) (width 0.2) (layer F.Cu) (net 9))
 (segment (start 165.645 82.92) (end 164 82.92) (width 0.2) (layer F.Cu) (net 10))
 (segment (start 168.473975 83.367172) (end 166.092172 83.367172) (width 0.2) (layer F.Cu) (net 10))
 (segment (start 166.092172 83.367172) (end 165.645 82.92) (width 0.2) (layer F.Cu) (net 10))
 (segment (start 178.15 88.35) (end 177.2 88.35) (width 0.2) (layer F.Cu) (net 20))
 (segment (start 178.5 88.7) (end 178.15 88.35) (width 0.2) (layer F.Cu) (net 20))
 (segment (start 178.5 89.2) (end 178.5 88.7) (width 0.2) (layer F.Cu) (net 20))
 (segment (start 181.3 91.8) (end 181.3 90.54) (width 0.2) (layer B.Cu) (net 20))
 (segment (start 178.9 89.6) (end 178.5 89.2) (width 0.2) (layer F.Cu) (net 20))
 (via (at 181.3 91.8) (size 0.4) (drill 0.254) (layers F.Cu B.Cu) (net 20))
 (segment (start 179.3 91.3) (end 179.3 90.8) (width 0.2) (layer F.Cu) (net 20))
 (segment (start 181.3 91.8) (end 179.8 91.8) (width 0.2) (layer F.Cu) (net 20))
 (segment (start 179.3 90.8) (end 178.9 90.4) (width 0.2) (layer F.Cu) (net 20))
 (segment (start 179.8 91.8) (end 179.3 91.3) (width 0.2) (layer F.Cu) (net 20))
 (segment (start 178.9 90.4) (end 178.9 89.6) (width 0.2) (layer F.Cu) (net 20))
 (segment (start 177.2 87.85) (end 178.25 87.85) (width 0.2) (layer F.Cu) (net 21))
 (segment (start 178.25 87.85) (end 178.9 88.5) (width 0.2) (layer F.Cu) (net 21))
 (segment (start 178.9 88.5) (end 178.9 89) (width 0.2) (layer F.Cu) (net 21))
 (segment (start 178.9 89) (end 179.3 89.4) (width 0.2) (layer F.Cu) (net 21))
 (segment (start 179.3 89.4) (end 179.3 90.2) (width 0.2) (layer F.Cu) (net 21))
 (segment (start 179.64 90.54) (end 181.3 90.54) (width 0.2) (layer F.Cu) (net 21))
 (segment (start 179.3 90.2) (end 179.64 90.54) (width 0.2) (layer F.Cu) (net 21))
 (segment (start 181.3 89.3) (end 181.3 88) (width 0.2) (layer B.Cu) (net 22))
 (via (at 181.3 89.3) (size 0.4) (drill 0.254) (layers F.Cu B.Cu) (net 22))
 (segment (start 178.35 87.35) (end 177.2 87.35) (width 0.2) (layer F.Cu) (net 22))
 (segment (start 179.3 88.3) (end 178.35 87.35) (width 0.2) (layer F.Cu) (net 22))
 (segment (start 179.3 88.8) (end 179.3 88.3) (width 0.2) (layer F.Cu) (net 22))
 (segment (start 181.3 89.3) (end 179.8 89.3) (width 0.2) (layer F.Cu) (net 22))
 (segment (start 179.8 89.3) (end 179.3 88.8) (width 0.2) (layer F.Cu) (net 22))
 (segment (start 179.6 88) (end 181.3 88) (width 0.2) (layer F.Cu) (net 23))
 (segment (start 177.2 86.85) (end 178.45 86.85) (width 0.2) (layer F.Cu) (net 23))
 (segment (start 178.45 86.85) (end 179.6 88) (width 0.2) (layer F.Cu) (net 23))
 (segment (start 181.3 86.75) (end 181.3 85.46) (width 0.2) (layer B.Cu) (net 24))
 (segment (start 178.95 85.75) (end 177.2 85.75) (width 0.2) (layer F.Cu) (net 24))
 (segment (start 179.95 86.75) (end 178.95 85.75) (width 0.2) (layer F.Cu) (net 24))
 (via (at 181.3 86.75) (size 0.4) (drill 0.254) (layers F.Cu B.Cu) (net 24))
 (segment (start 181.3 86.75) (end 179.95 86.75) (width 0.2) (layer F.Cu) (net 24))
 (segment (start 177.2 85.25) (end 179.45 85.25) (width 0.2) (layer F.Cu) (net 25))
 (segment (start 179.66 85.46) (end 181.3 85.46) (width 0.2) (layer F.Cu) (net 25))
 (segment (start 179.45 85.25) (end 179.66 85.46) (width 0.2) (layer F.Cu) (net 25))
 (segment (start 181.35 84.2) (end 181.3 84.15) (width 0.2) (layer B.Cu) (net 26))
 (segment (start 178.25 84.75) (end 177.2 84.75) (width 0.2) (layer F.Cu) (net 26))
 (segment (start 178.8 84.2) (end 178.25 84.75) (width 0.2) (layer F.Cu) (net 26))
 (segment (start 181.3 84.15) (end 181.3 82.92) (width 0.2) (layer B.Cu) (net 26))
 (via (at 181.35 84.2) (size 0.4) (drill 0.254) (layers F.Cu B.Cu) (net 26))
 (segment (start 181.35 84.2) (end 178.8 84.2) (width 0.2) (layer F.Cu) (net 26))
 (segment (start 177.2 84.25) (end 178.25 84.25) (width 0.2) (layer F.Cu) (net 27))
 (segment (start 179.58 82.92) (end 181.3 82.92) (width 0.2) (layer F.Cu) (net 27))
 (segment (start 178.25 84.25) (end 179.58 82.92) (width 0.2) (layer F.Cu) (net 27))
 (segment (start 175.8 85.75) (end 176.2 85.75) (width 0.2) (layer F.Cu) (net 14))
 (segment (start 174.323975 85.967172) (end 175.582828 85.967172) (width 0.2) (layer F.Cu) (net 14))
 (segment (start 175.582828 85.967172) (end 175.8 85.75) (width 0.2) (layer F.Cu) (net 14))
 (segment (start 174.323975 84.667172) (end 175.667172 84.667172) (width 0.2) (layer F.Cu) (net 12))
 (segment (start 175.75 84.75) (end 176.2 84.75) (width 0.2) (layer F.Cu) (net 12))
 (segment (start 175.667172 84.667172) (end 175.75 84.75) (width 0.2) (layer F.Cu) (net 12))
 (segment (start 175.75 85.25) (end 176.2 85.25) (width 0.2) (layer F.Cu) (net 13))
 (segment (start 174.323975 85.317172) (end 175.682828 85.317172) (width 0.2) (layer F.Cu) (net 13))
 (segment (start 175.682828 85.317172) (end 175.75 85.25) (width 0.2) (layer F.Cu) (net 13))
 (segment (start 174.323975 84.017172) (end 175.567172 84.017172) (width 0.2) (layer F.Cu) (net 11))
 (segment (start 175.8 84.25) (end 176.2 84.25) (width 0.2) (layer F.Cu) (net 11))
 (segment (start 175.567172 84.017172) (end 175.8 84.25) (width 0.2) (layer F.Cu) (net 11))
 (segment (start 175.8 88.35) (end 176.2 88.35) (width 0.2) (layer F.Cu) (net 18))
 (segment (start 174.323975 88.567172) (end 175.582828 88.567172) (width 0.2) (layer F.Cu) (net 18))
 (segment (start 175.582828 88.567172) (end 175.8 88.35) (width 0.2) (layer F.Cu) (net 18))
 (segment (start 175.8 87.35) (end 176.2 87.35) (width 0.2) (layer F.Cu) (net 16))
 (segment (start 174.323975 87.267172) (end 175.717172 87.267172) (width 0.2) (layer F.Cu) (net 16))
 (segment (start 175.717172 87.267172) (end 175.8 87.35) (width 0.2) (layer F.Cu) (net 16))
 (segment (start 175.8 87.85) (end 176.2 87.85) (width 0.2) (layer F.Cu) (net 17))
 (segment (start 174.323975 87.917172) (end 175.732828 87.917172) (width 0.2) (layer F.Cu) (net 17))
 (segment (start 175.732828 87.917172) (end 175.8 87.85) (width 0.2) (layer F.Cu) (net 17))
 (segment (start 175.8 86.85) (end 176.2 86.85) (width 0.2) (layer F.Cu) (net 15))
 (segment (start 174.323975 86.617172) (end 175.567172 86.617172) (width 0.2) (layer F.Cu) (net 15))
 (segment (start 175.567172 86.617172) (end 175.8 86.85) (width 0.2) (layer F.Cu) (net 15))
 (segment (start 171.5 92.45) (end 172.05 92.45) (width 0.2) (layer F.Cu) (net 30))
 (segment (start 172.2 92.6) (end 172.7 92.6) (width 0.2) (layer F.Cu) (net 30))
 (segment (start 172.05 92.45) (end 172.2 92.6) (width 0.2) (layer F.Cu) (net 30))
 (segment (start 176 92.3) (end 176 91.8) (width 0.2) (layer F.Cu) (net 29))
 (segment (start 175.8 92.5) (end 176 92.3) (width 0.2) (layer F.Cu) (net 29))
 (segment (start 175.8 92.9) (end 175.8 92.5) (width 0.2) (layer F.Cu) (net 29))
 (segment (start 175 93.05) (end 175.65 93.05) (width 0.2) (layer F.Cu) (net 29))
 (segment (start 175.65 93.05) (end 175.8 92.9) (width 0.2) (layer F.Cu) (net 29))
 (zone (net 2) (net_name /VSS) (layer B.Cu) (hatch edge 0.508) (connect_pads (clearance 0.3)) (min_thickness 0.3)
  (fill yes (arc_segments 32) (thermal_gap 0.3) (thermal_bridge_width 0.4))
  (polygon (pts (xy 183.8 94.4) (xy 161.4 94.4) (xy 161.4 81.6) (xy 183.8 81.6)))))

